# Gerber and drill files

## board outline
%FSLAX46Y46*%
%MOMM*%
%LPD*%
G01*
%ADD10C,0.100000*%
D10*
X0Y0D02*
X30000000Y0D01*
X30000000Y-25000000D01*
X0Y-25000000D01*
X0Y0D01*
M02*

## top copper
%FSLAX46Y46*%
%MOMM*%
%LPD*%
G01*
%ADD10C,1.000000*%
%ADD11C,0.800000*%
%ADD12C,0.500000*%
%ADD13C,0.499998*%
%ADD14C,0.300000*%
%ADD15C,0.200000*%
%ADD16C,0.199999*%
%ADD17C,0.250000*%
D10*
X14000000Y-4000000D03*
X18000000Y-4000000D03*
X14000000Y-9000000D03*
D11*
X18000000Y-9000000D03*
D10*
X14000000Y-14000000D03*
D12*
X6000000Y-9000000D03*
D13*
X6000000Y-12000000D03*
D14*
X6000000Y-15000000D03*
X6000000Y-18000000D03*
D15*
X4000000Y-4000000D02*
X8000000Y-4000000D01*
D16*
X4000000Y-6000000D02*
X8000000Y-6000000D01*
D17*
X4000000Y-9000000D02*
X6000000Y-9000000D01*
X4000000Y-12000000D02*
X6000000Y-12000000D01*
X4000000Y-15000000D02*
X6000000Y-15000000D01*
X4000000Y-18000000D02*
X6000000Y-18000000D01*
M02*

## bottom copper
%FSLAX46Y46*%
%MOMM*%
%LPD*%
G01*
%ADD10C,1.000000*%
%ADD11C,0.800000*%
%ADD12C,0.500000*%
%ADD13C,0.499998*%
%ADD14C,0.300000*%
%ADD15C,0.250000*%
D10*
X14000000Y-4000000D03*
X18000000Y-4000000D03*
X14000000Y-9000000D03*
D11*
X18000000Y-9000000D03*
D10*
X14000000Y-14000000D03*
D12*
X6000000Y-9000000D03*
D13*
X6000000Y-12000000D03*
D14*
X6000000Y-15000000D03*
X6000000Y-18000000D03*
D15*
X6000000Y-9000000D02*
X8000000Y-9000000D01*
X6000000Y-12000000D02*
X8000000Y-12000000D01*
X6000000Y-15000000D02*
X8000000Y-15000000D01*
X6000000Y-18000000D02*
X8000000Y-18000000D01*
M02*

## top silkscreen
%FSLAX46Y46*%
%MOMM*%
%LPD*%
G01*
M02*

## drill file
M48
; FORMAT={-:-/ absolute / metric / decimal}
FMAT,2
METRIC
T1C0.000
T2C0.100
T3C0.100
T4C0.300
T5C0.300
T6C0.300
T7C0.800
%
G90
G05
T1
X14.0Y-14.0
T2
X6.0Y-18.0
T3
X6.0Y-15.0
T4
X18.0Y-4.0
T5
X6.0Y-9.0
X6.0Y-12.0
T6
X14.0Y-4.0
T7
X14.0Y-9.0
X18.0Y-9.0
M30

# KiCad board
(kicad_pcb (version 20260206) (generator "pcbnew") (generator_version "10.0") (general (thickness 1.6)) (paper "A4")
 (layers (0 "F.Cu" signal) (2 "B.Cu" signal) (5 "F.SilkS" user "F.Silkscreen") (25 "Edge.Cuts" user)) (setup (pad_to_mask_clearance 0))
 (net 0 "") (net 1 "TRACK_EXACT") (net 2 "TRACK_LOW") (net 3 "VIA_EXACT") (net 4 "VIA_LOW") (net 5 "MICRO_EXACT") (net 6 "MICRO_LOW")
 (segment (start 4 4) (end 8 4) (width 0.2) (layer "F.Cu") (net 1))
 (segment (start 4 6) (end 8 6) (width 0.199999) (layer "F.Cu") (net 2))
 (segment (start 4 9) (end 6 9) (width 0.25) (layer "F.Cu") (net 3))
 (via (at 6 9) (size 0.5) (drill 0.3) (layers "F.Cu" "B.Cu") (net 3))
 (segment (start 6 9) (end 8 9) (width 0.25) (layer "B.Cu") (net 3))
 (segment (start 4 12) (end 6 12) (width 0.25) (layer "F.Cu") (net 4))
 (via (at 6 12) (size 0.499998) (drill 0.3) (layers "F.Cu" "B.Cu") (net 4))
 (segment (start 6 12) (end 8 12) (width 0.25) (layer "B.Cu") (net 4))
 (segment (start 4 15) (end 6 15) (width 0.25) (layer "F.Cu") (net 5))
 (via micro (at 6 15) (size 0.3) (drill 0.1) (layers "F.Cu" "B.Cu") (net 5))
 (segment (start 6 15) (end 8 15) (width 0.25) (layer "B.Cu") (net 5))
 (segment (start 4 18) (end 6 18) (width 0.25) (layer "F.Cu") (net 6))
 (via micro (at 6 18) (size 0.3) (drill 0.099999) (layers "F.Cu" "B.Cu") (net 6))
 (segment (start 6 18) (end 8 18) (width 0.25) (layer "B.Cu") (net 6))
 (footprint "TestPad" (layer "F.Cu") (at 14 4)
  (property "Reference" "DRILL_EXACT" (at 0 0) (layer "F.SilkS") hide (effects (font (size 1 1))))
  (pad "1" thru_hole circle (at 0 0) (size 1 1) (drill 0.3) (layers "*.Cu" "*.Mask")))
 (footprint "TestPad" (layer "F.Cu") (at 18 4)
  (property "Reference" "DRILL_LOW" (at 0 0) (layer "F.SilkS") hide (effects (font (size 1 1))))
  (pad "1" thru_hole circle (at 0 0) (size 1 1) (drill 0.299999) (layers "*.Cu" "*.Mask")))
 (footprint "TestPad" (layer "F.Cu") (at 14 9)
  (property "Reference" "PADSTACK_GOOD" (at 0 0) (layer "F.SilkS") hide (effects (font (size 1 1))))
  (pad "1" thru_hole circle (at 0 0) (size 1 1) (drill 0.8) (layers "*.Cu" "*.Mask")))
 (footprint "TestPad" (layer "F.Cu") (at 18 9)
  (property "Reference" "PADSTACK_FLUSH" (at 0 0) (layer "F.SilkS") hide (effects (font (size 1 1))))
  (pad "1" thru_hole circle (at 0 0) (size 0.8 0.8) (drill 0.8) (layers "*.Cu" "*.Mask")))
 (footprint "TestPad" (layer "F.Cu") (at 14 14)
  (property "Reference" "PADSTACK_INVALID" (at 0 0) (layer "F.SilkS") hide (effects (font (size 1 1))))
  (pad "1" thru_hole circle (at 0 0) (size 1 1) (layers "*.Cu" "*.Mask")))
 (gr_rect (start 0 0) (end 30 25) (stroke (width 0.1) (type default)) (fill no) (layer "Edge.Cuts")))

